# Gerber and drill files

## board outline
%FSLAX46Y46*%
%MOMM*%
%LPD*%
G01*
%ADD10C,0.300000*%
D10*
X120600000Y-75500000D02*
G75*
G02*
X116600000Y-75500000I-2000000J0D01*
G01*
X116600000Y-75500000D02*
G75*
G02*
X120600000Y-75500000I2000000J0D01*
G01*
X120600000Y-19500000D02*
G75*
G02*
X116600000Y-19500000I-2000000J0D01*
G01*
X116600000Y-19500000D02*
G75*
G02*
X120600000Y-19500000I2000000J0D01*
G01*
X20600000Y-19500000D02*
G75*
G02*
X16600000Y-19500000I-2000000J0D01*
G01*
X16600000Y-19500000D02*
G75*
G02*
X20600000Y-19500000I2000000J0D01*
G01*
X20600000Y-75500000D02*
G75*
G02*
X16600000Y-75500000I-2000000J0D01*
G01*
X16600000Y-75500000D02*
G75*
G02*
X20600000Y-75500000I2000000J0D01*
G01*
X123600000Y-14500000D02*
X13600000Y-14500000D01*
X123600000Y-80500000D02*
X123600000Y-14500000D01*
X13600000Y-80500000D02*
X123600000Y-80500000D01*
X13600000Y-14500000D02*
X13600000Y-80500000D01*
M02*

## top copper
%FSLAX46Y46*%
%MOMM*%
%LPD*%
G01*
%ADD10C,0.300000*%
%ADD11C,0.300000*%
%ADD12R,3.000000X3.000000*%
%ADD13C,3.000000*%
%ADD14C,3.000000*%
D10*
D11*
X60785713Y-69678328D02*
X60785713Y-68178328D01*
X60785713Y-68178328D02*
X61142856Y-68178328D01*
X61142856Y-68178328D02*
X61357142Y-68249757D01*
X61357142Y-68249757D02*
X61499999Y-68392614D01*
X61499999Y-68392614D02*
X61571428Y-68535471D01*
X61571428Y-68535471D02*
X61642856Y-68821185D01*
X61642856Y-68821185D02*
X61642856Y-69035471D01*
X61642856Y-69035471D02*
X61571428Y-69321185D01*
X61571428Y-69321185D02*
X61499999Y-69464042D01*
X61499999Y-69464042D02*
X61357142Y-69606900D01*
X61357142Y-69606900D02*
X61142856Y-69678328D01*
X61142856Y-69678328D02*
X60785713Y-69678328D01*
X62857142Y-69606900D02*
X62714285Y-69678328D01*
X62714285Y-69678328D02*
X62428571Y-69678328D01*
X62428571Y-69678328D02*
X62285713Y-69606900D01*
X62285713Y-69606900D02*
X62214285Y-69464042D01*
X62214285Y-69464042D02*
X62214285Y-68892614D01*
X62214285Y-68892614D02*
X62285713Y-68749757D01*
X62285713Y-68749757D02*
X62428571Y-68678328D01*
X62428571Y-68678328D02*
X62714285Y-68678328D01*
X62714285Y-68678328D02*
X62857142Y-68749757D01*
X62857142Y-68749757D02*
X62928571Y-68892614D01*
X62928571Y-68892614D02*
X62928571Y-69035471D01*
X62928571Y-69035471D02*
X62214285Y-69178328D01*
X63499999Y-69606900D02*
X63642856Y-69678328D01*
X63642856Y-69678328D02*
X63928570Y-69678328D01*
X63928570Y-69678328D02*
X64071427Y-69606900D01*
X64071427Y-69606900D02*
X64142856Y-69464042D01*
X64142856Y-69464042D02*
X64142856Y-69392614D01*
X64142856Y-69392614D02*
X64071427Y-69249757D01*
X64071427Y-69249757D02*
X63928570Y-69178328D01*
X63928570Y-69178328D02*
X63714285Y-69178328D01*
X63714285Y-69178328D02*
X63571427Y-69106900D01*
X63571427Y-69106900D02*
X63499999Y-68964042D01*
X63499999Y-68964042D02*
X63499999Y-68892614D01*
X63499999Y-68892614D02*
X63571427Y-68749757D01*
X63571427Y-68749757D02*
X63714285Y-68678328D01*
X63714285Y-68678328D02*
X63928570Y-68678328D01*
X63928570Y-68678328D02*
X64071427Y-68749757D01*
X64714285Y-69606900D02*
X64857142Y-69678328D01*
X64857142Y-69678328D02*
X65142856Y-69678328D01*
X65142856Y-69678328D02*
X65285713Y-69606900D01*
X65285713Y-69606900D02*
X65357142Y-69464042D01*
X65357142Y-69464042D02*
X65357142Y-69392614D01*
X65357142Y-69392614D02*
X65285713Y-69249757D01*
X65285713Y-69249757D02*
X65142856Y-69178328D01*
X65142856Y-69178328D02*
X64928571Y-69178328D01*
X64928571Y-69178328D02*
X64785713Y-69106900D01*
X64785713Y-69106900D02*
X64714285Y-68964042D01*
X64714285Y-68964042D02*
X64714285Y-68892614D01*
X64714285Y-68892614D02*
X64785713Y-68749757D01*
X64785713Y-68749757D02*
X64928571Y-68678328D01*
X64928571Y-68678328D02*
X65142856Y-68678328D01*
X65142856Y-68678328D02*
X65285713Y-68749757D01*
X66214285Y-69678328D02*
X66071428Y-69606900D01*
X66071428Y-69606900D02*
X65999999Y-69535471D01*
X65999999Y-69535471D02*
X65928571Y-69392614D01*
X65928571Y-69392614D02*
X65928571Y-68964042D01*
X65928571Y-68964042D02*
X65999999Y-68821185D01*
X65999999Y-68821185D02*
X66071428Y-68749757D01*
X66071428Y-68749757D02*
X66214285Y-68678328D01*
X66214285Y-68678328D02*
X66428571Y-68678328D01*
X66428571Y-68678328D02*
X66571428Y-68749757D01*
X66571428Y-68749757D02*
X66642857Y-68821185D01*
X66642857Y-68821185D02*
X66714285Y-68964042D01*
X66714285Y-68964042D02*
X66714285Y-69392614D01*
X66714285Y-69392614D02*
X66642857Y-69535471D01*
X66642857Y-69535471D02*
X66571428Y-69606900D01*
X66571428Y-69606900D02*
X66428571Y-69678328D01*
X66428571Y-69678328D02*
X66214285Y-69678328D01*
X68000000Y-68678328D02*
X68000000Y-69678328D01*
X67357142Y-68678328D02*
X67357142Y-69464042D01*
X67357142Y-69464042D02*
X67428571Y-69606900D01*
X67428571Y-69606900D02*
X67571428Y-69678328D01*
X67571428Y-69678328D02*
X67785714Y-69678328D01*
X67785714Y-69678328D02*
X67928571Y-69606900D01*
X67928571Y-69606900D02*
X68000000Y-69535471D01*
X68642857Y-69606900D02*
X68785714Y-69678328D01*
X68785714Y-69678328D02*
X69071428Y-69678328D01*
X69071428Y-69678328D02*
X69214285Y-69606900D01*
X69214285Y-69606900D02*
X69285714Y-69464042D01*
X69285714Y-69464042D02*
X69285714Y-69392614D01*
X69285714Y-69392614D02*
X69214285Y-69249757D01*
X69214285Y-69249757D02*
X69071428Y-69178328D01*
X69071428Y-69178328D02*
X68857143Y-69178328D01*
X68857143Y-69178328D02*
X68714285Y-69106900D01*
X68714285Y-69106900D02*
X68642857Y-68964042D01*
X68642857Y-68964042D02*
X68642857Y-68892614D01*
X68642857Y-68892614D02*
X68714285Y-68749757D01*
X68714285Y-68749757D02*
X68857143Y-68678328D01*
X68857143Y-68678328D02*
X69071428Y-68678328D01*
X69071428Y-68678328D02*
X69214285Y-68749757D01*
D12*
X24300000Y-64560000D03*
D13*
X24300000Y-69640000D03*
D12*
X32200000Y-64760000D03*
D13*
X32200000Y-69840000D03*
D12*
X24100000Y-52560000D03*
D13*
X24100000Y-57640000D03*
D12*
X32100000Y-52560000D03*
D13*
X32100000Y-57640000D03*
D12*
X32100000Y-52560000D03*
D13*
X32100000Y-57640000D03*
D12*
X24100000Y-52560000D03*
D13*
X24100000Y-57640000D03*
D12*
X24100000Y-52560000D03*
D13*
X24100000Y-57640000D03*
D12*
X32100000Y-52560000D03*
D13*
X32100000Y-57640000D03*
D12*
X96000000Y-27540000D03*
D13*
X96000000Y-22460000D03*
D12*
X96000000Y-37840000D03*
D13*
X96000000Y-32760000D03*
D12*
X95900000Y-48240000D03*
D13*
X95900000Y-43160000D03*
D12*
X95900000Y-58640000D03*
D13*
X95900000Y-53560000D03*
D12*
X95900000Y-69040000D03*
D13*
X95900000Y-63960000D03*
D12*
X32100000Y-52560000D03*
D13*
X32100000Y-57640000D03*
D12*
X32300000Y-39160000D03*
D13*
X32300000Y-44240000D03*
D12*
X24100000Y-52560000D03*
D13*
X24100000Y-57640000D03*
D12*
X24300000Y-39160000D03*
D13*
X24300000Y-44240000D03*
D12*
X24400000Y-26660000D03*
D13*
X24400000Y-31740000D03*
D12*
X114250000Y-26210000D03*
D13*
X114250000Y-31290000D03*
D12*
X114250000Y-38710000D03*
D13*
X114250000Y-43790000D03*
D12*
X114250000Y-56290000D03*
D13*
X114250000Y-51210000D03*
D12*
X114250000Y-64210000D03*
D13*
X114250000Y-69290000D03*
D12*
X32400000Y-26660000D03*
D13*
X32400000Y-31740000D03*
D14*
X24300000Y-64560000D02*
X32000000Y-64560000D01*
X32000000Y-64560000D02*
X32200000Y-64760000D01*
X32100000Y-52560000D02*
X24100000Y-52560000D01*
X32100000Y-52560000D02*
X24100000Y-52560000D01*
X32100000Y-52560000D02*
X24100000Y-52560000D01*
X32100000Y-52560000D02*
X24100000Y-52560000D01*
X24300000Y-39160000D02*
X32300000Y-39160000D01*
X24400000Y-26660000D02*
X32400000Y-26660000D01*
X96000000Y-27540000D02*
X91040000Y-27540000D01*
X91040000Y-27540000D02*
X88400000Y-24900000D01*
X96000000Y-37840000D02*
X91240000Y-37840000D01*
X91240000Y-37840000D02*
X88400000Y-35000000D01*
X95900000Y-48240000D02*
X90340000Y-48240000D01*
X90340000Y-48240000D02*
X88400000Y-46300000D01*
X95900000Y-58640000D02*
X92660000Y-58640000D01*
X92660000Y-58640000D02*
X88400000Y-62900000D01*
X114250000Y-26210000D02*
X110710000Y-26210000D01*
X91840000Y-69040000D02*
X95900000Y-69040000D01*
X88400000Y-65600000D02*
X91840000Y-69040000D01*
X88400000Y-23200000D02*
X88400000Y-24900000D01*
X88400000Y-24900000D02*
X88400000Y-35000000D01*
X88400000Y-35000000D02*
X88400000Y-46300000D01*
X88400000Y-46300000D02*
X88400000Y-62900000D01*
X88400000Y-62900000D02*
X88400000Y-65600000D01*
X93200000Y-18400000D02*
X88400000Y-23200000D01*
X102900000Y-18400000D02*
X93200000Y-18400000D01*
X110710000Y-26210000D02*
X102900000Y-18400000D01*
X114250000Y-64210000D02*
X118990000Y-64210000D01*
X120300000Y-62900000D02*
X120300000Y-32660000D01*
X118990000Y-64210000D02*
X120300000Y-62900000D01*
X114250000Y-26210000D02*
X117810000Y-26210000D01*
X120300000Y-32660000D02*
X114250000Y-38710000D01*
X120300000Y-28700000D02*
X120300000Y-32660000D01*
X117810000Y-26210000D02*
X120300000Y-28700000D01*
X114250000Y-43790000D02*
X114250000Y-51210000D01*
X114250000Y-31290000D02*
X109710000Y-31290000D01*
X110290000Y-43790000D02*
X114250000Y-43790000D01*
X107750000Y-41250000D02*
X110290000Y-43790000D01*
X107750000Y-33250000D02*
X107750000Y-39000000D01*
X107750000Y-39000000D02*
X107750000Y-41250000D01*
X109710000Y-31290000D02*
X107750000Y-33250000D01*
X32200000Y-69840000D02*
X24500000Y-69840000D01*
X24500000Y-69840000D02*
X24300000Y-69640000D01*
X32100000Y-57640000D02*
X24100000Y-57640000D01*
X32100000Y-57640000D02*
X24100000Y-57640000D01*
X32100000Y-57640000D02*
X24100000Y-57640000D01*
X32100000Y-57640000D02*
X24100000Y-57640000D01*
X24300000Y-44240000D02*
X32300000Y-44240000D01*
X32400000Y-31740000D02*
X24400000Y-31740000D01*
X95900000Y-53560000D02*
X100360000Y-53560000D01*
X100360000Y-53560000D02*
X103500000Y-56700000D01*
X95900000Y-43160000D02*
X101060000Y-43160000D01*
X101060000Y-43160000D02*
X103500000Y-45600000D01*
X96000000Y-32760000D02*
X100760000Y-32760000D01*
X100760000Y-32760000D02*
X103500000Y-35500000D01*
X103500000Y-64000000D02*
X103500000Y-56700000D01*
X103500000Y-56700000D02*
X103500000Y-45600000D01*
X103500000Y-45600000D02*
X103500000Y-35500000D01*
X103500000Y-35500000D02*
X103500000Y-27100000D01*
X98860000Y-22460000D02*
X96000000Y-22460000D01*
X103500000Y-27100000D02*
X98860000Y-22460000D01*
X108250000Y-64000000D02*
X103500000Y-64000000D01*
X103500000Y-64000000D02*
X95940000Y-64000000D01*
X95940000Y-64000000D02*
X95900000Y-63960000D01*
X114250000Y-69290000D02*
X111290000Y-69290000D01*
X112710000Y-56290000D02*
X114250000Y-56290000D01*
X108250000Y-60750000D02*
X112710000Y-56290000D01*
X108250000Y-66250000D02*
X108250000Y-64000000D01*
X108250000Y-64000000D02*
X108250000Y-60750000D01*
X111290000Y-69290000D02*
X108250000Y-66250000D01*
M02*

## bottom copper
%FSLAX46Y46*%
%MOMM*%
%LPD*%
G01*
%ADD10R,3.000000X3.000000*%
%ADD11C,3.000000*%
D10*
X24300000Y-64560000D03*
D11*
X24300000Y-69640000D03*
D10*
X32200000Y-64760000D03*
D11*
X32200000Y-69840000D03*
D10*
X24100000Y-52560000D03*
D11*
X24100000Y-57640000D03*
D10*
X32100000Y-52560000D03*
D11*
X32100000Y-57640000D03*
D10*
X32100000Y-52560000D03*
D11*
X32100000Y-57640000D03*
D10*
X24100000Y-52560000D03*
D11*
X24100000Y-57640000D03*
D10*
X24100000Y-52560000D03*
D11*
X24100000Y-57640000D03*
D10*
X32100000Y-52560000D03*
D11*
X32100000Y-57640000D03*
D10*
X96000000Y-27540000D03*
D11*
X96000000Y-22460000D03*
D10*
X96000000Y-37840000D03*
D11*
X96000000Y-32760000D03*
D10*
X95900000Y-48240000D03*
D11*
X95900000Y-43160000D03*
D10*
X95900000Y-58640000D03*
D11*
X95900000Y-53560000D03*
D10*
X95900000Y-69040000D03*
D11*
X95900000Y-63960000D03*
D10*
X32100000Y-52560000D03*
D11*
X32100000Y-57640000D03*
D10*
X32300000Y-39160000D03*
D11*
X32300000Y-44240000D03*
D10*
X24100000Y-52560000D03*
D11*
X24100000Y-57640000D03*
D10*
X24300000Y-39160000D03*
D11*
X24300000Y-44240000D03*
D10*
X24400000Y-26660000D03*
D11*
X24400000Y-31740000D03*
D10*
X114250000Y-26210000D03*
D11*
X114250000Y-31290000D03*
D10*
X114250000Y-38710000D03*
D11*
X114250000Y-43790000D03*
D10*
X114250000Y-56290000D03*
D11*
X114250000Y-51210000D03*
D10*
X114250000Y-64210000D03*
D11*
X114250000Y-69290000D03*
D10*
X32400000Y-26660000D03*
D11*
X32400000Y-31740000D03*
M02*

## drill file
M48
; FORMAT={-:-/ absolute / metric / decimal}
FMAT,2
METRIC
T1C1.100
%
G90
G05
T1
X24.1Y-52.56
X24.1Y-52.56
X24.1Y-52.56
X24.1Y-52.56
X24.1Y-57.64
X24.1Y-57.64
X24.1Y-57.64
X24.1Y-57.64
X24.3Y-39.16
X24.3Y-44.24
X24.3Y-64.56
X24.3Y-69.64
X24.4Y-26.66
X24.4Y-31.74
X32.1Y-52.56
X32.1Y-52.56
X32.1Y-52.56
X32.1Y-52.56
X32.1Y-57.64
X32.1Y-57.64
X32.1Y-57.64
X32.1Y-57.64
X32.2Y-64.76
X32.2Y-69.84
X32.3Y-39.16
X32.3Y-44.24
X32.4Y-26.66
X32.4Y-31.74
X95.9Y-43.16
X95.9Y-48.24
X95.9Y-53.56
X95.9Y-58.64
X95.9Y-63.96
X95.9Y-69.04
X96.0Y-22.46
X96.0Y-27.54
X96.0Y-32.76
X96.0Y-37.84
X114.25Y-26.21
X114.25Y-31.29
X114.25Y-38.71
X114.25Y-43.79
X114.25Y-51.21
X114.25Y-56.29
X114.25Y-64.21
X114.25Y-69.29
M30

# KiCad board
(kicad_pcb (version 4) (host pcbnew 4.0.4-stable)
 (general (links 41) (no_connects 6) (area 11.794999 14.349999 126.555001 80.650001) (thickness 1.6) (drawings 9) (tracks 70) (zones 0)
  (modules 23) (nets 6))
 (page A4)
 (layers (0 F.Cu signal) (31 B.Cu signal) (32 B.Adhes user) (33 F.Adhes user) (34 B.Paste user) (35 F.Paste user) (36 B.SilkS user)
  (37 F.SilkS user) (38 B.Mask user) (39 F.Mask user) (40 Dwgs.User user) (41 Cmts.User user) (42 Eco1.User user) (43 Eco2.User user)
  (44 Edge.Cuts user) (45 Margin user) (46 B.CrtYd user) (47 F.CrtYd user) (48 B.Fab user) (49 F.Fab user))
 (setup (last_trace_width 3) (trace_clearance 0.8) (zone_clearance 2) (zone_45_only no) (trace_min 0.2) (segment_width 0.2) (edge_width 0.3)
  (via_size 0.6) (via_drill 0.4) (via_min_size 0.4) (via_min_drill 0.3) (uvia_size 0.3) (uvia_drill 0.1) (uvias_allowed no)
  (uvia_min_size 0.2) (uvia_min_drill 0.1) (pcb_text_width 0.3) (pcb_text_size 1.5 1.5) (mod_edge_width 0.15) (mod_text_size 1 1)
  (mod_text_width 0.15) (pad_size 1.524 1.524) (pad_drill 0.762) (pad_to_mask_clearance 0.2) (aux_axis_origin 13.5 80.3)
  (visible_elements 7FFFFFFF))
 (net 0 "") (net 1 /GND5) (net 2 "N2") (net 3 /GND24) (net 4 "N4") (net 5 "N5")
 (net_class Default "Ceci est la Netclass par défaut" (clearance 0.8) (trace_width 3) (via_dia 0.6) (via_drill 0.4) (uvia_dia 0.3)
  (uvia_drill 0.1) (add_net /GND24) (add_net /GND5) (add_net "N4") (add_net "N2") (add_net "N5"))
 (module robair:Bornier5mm (layer B.Cu) (at 24.3 67.1 270)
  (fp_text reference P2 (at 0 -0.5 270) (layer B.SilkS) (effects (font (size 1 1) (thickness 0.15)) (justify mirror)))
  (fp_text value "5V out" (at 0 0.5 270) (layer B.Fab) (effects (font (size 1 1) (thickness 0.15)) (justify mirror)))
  (pad 1 thru_hole rect (at -2.54 0 270) (size 3 3) (drill 1.1) (layers *.Cu *.Mask) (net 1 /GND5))
  (pad 2 thru_hole circle (at 2.54 0 270) (size 3 3) (drill 1.1) (layers *.Cu *.Mask) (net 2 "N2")))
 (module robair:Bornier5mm (layer F.Cu) (at 32.2 67.3 270)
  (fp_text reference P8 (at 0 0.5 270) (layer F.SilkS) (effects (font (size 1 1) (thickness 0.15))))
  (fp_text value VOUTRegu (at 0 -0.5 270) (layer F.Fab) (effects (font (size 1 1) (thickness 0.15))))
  (pad 1 thru_hole rect (at -2.54 0 270) (size 3 3) (drill 1.1) (layers *.Cu *.Mask) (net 1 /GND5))
  (pad 2 thru_hole circle (at 2.54 0 270) (size 3 3) (drill 1.1) (layers *.Cu *.Mask) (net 2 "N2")))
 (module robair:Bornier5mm (layer B.Cu) (at 24.1 55.1 270)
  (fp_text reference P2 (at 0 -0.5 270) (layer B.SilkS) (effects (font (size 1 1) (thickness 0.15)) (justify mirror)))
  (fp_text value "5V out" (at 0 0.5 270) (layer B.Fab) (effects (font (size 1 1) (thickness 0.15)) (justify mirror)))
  (pad 1 thru_hole rect (at -2.54 0 270) (size 3 3) (drill 1.1) (layers *.Cu *.Mask) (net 1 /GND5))
  (pad 2 thru_hole circle (at 2.54 0 270) (size 3 3) (drill 1.1) (layers *.Cu *.Mask) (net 2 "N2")))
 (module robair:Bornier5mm (layer F.Cu) (at 32.1 55.1 270)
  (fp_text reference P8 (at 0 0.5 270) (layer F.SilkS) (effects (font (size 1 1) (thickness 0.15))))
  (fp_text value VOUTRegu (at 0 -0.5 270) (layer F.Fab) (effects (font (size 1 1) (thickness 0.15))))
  (pad 1 thru_hole rect (at -2.54 0 270) (size 3 3) (drill 1.1) (layers *.Cu *.Mask) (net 1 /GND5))
  (pad 2 thru_hole circle (at 2.54 0 270) (size 3 3) (drill 1.1) (layers *.Cu *.Mask) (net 2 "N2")))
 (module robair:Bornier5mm (layer F.Cu) (at 32.1 55.1 270)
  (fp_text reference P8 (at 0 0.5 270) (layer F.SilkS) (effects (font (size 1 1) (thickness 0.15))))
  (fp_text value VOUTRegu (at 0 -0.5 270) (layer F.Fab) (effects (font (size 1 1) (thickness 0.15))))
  (pad 1 thru_hole rect (at -2.54 0 270) (size 3 3) (drill 1.1) (layers *.Cu *.Mask) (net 1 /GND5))
  (pad 2 thru_hole circle (at 2.54 0 270) (size 3 3) (drill 1.1) (layers *.Cu *.Mask) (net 2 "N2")))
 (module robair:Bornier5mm (layer B.Cu) (at 24.1 55.1 270)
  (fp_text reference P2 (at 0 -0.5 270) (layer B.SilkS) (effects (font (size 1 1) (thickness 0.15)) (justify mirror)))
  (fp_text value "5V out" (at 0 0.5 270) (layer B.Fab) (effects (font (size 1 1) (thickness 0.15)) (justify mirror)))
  (pad 1 thru_hole rect (at -2.54 0 270) (size 3 3) (drill 1.1) (layers *.Cu *.Mask) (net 1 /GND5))
  (pad 2 thru_hole circle (at 2.54 0 270) (size 3 3) (drill 1.1) (layers *.Cu *.Mask) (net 2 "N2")))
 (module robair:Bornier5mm (layer B.Cu) (at 24.1 55.1 270)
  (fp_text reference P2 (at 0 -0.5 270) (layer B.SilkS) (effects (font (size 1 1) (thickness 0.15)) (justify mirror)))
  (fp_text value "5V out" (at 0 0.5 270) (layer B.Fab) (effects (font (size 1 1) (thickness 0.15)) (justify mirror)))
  (pad 1 thru_hole rect (at -2.54 0 270) (size 3 3) (drill 1.1) (layers *.Cu *.Mask) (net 1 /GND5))
  (pad 2 thru_hole circle (at 2.54 0 270) (size 3 3) (drill 1.1) (layers *.Cu *.Mask) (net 2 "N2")))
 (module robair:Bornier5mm (layer F.Cu) (at 32.1 55.1 270)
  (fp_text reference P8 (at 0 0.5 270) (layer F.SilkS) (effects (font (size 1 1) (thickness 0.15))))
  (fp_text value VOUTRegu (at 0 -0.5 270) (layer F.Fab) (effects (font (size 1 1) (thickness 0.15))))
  (pad 1 thru_hole rect (at -2.54 0 270) (size 3 3) (drill 1.1) (layers *.Cu *.Mask) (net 1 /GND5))
  (pad 2 thru_hole circle (at 2.54 0 270) (size 3 3) (drill 1.1) (layers *.Cu *.Mask) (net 2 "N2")))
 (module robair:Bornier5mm (layer F.Cu) (at 96 25 90)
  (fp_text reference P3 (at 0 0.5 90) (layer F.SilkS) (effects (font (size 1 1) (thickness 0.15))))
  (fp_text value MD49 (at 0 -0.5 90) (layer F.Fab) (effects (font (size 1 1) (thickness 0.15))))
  (pad 1 thru_hole rect (at -2.54 0 90) (size 3 3) (drill 1.1) (layers *.Cu *.Mask) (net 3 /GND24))
  (pad 2 thru_hole circle (at 2.54 0 90) (size 3 3) (drill 1.1) (layers *.Cu *.Mask) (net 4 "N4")))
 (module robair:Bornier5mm (layer F.Cu) (at 96 35.3 90)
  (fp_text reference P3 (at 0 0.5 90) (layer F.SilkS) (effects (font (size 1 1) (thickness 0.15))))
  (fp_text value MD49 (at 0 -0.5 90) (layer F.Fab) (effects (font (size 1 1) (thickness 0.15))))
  (pad 1 thru_hole rect (at -2.54 0 90) (size 3 3) (drill 1.1) (layers *.Cu *.Mask) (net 3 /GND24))
  (pad 2 thru_hole circle (at 2.54 0 90) (size 3 3) (drill 1.1) (layers *.Cu *.Mask) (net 4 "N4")))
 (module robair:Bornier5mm (layer F.Cu) (at 95.9 45.7 90)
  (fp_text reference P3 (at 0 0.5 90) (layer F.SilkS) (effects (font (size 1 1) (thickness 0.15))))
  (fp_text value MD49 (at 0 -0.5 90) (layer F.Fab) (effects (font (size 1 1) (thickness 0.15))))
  (pad 1 thru_hole rect (at -2.54 0 90) (size 3 3) (drill 1.1) (layers *.Cu *.Mask) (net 3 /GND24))
  (pad 2 thru_hole circle (at 2.54 0 90) (size 3 3) (drill 1.1) (layers *.Cu *.Mask) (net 4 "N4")))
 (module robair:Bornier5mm (layer F.Cu) (at 95.9 56.1 90)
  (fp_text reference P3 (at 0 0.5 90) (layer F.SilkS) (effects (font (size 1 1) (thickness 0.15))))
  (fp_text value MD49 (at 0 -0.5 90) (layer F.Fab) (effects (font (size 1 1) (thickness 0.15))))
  (pad 1 thru_hole rect (at -2.54 0 90) (size 3 3) (drill 1.1) (layers *.Cu *.Mask) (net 3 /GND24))
  (pad 2 thru_hole circle (at 2.54 0 90) (size 3 3) (drill 1.1) (layers *.Cu *.Mask) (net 4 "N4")))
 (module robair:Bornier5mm (layer F.Cu) (at 95.9 66.5 90)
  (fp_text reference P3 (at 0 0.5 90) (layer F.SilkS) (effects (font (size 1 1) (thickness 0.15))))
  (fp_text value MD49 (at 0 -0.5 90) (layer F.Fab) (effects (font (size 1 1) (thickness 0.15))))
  (pad 1 thru_hole rect (at -2.54 0 90) (size 3 3) (drill 1.1) (layers *.Cu *.Mask) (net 3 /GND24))
  (pad 2 thru_hole circle (at 2.54 0 90) (size 3 3) (drill 1.1) (layers *.Cu *.Mask) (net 4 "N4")))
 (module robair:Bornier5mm (layer F.Cu) (at 32.1 55.1 270)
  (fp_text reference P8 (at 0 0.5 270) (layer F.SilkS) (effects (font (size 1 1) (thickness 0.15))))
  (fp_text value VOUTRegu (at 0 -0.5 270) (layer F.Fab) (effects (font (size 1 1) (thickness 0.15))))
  (pad 1 thru_hole rect (at -2.54 0 270) (size 3 3) (drill 1.1) (layers *.Cu *.Mask) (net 1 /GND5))
  (pad 2 thru_hole circle (at 2.54 0 270) (size 3 3) (drill 1.1) (layers *.Cu *.Mask) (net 2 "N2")))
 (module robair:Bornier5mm (layer F.Cu) (at 32.3 41.7 270)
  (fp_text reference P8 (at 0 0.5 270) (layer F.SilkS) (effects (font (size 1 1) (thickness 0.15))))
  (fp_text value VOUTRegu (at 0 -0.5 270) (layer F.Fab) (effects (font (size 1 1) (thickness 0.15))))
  (pad 1 thru_hole rect (at -2.54 0 270) (size 3 3) (drill 1.1) (layers *.Cu *.Mask) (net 1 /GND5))
  (pad 2 thru_hole circle (at 2.54 0 270) (size 3 3) (drill 1.1) (layers *.Cu *.Mask) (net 2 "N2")))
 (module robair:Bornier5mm (layer B.Cu) (at 24.1 55.1 270)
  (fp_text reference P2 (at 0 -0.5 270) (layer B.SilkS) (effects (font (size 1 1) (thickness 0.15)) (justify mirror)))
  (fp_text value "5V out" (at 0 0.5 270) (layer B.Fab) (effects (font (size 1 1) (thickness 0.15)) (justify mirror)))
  (pad 1 thru_hole rect (at -2.54 0 270) (size 3 3) (drill 1.1) (layers *.Cu *.Mask) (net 1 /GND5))
  (pad 2 thru_hole circle (at 2.54 0 270) (size 3 3) (drill 1.1) (layers *.Cu *.Mask) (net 2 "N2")))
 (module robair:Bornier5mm (layer B.Cu) (at 24.3 41.7 270)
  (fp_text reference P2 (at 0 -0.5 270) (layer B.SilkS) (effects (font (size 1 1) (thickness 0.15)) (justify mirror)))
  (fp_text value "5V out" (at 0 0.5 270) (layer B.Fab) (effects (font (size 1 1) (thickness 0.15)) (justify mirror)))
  (pad 1 thru_hole rect (at -2.54 0 270) (size 3 3) (drill 1.1) (layers *.Cu *.Mask) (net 1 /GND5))
  (pad 2 thru_hole circle (at 2.54 0 270) (size 3 3) (drill 1.1) (layers *.Cu *.Mask) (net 2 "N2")))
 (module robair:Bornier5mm (layer B.Cu) (at 24.4 29.2 270)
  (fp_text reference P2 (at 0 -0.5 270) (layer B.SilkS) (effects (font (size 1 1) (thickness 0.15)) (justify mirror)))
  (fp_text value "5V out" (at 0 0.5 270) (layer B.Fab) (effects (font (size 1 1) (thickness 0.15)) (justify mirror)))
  (pad 1 thru_hole rect (at -2.54 0 270) (size 3 3) (drill 1.1) (layers *.Cu *.Mask) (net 1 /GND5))
  (pad 2 thru_hole circle (at 2.54 0 270) (size 3 3) (drill 1.1) (layers *.Cu *.Mask) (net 2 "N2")))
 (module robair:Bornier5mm (layer F.Cu) (at 114.25 28.75 270)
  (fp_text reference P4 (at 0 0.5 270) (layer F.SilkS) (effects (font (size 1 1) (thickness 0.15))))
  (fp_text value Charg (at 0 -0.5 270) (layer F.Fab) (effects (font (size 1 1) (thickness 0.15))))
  (pad 1 thru_hole rect (at -2.54 0 270) (size 3 3) (drill 1.1) (layers *.Cu *.Mask) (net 3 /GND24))
  (pad 2 thru_hole circle (at 2.54 0 270) (size 3 3) (drill 1.1) (layers *.Cu *.Mask) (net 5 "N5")))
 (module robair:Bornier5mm (layer F.Cu) (at 114.25 41.25 270)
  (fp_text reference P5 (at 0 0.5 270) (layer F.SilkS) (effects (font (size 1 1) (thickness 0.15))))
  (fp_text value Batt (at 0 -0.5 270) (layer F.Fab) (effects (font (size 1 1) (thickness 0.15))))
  (pad 1 thru_hole rect (at -2.54 0 270) (size 3 3) (drill 1.1) (layers *.Cu *.Mask) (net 3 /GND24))
  (pad 2 thru_hole circle (at 2.54 0 270) (size 3 3) (drill 1.1) (layers *.Cu *.Mask) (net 5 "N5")))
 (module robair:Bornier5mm (layer B.Cu) (at 114.25 53.75 90)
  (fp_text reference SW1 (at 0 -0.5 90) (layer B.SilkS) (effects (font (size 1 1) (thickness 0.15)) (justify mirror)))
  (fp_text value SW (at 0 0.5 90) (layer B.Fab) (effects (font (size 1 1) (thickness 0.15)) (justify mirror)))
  (pad 1 thru_hole rect (at -2.54 0 90) (size 3 3) (drill 1.1) (layers *.Cu *.Mask) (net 4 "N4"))
  (pad 2 thru_hole circle (at 2.54 0 90) (size 3 3) (drill 1.1) (layers *.Cu *.Mask) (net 5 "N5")))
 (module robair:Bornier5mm (layer F.Cu) (at 114.25 66.75 270)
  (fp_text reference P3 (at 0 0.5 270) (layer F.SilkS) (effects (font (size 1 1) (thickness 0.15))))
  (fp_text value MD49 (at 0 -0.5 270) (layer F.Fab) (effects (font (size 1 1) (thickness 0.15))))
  (pad 1 thru_hole rect (at -2.54 0 270) (size 3 3) (drill 1.1) (layers *.Cu *.Mask) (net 3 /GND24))
  (pad 2 thru_hole circle (at 2.54 0 270) (size 3 3) (drill 1.1) (layers *.Cu *.Mask) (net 4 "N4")))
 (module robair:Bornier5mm (layer F.Cu) (at 32.4 29.2 270)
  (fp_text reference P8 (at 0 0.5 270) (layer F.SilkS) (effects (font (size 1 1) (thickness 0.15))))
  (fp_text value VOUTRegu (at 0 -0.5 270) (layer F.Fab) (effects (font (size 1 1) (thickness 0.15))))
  (pad 1 thru_hole rect (at -2.54 0 270) (size 3 3) (drill 1.1) (layers *.Cu *.Mask) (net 1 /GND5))
  (pad 2 thru_hole circle (at 2.54 0 270) (size 3 3) (drill 1.1) (layers *.Cu *.Mask) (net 2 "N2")))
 (gr_circle (center 118.6 75.5) (end 118.6 77.5) (layer Edge.Cuts) (width 0.3))
 (gr_circle (center 118.6 19.5) (end 120.6 19.5) (layer Edge.Cuts) (width 0.3))
 (gr_circle (center 18.6 19.5) (end 16.6 19.5) (layer Edge.Cuts) (width 0.3))
 (gr_circle (center 18.6 75.5) (end 16.6 75.5) (layer Edge.Cuts) (width 0.3))
 (gr_line (start 123.6 14.5) (end 13.6 14.5) (angle 90) (layer Edge.Cuts) (width 0.3))
 (gr_line (start 123.6 80.5) (end 123.6 14.5) (angle 90) (layer Edge.Cuts) (width 0.3))
 (gr_line (start 13.6 80.5) (end 123.6 80.5) (angle 90) (layer Edge.Cuts) (width 0.3))
 (gr_line (start 13.6 14.5) (end 13.6 80.5) (angle 90) (layer Edge.Cuts) (width 0.3))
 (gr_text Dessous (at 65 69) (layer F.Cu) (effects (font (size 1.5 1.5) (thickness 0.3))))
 (segment (start 24.3 64.56) (end 32 64.56) (width 3) (layer F.Cu) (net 1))
 (segment (start 32 64.56) (end 32.2 64.76) (width 3) (layer F.Cu) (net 1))
 (segment (start 32.1 52.56) (end 24.1 52.56) (width 3) (layer F.Cu) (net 1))
 (segment (start 32.1 52.56) (end 24.1 52.56) (width 3) (layer F.Cu) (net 1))
 (segment (start 32.1 52.56) (end 24.1 52.56) (width 3) (layer F.Cu) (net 1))
 (segment (start 32.1 52.56) (end 24.1 52.56) (width 3) (layer F.Cu) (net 1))
 (segment (start 24.3 39.16) (end 32.3 39.16) (width 3) (layer F.Cu) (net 1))
 (segment (start 24.4 26.66) (end 32.4 26.66) (width 3) (layer F.Cu) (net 1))
 (segment (start 96 27.54) (end 91.04 27.54) (width 3) (layer F.Cu) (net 3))
 (segment (start 91.04 27.54) (end 88.4 24.9) (width 3) (layer F.Cu) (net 3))
 (segment (start 96 37.84) (end 91.24 37.84) (width 3) (layer F.Cu) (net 3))
 (segment (start 91.24 37.84) (end 88.4 35) (width 3) (layer F.Cu) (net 3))
 (segment (start 95.9 48.24) (end 90.34 48.24) (width 3) (layer F.Cu) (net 3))
 (segment (start 90.34 48.24) (end 88.4 46.3) (width 3) (layer F.Cu) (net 3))
 (segment (start 95.9 58.64) (end 92.66 58.64) (width 3) (layer F.Cu) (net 3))
 (segment (start 92.66 58.64) (end 88.4 62.9) (width 3) (layer F.Cu) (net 3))
 (segment (start 114.25 26.21) (end 110.71 26.21) (width 3) (layer F.Cu) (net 3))
 (segment (start 91.84 69.04) (end 95.9 69.04) (width 3) (layer F.Cu) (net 3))
 (segment (start 88.4 65.6) (end 91.84 69.04) (width 3) (layer F.Cu) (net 3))
 (segment (start 88.4 23.2) (end 88.4 24.9) (width 3) (layer F.Cu) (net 3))
 (segment (start 88.4 24.9) (end 88.4 35) (width 3) (layer F.Cu) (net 3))
 (segment (start 88.4 35) (end 88.4 46.3) (width 3) (layer F.Cu) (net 3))
 (segment (start 88.4 46.3) (end 88.4 62.9) (width 3) (layer F.Cu) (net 3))
 (segment (start 88.4 62.9) (end 88.4 65.6) (width 3) (layer F.Cu) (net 3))
 (segment (start 93.2 18.4) (end 88.4 23.2) (width 3) (layer F.Cu) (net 3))
 (segment (start 102.9 18.4) (end 93.2 18.4) (width 3) (layer F.Cu) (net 3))
 (segment (start 110.71 26.21) (end 102.9 18.4) (width 3) (layer F.Cu) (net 3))
 (segment (start 114.25 64.21) (end 118.99 64.21) (width 3) (layer F.Cu) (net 3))
 (segment (start 120.3 62.9) (end 120.3 32.66) (width 3) (layer F.Cu) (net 3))
 (segment (start 118.99 64.21) (end 120.3 62.9) (width 3) (layer F.Cu) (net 3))
 (segment (start 114.25 26.21) (end 117.81 26.21) (width 3) (layer F.Cu) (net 3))
 (segment (start 120.3 32.66) (end 114.25 38.71) (width 3) (layer F.Cu) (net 3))
 (segment (start 120.3 28.7) (end 120.3 32.66) (width 3) (layer F.Cu) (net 3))
 (segment (start 117.81 26.21) (end 120.3 28.7) (width 3) (layer F.Cu) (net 3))
 (segment (start 114.25 43.79) (end 114.25 51.21) (width 3) (layer F.Cu) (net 5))
 (segment (start 114.25 31.29) (end 109.71 31.29) (width 3) (layer F.Cu) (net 5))
 (segment (start 110.29 43.79) (end 114.25 43.79) (width 3) (layer F.Cu) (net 5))
 (segment (start 107.75 41.25) (end 110.29 43.79) (width 3) (layer F.Cu) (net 5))
 (segment (start 107.75 33.25) (end 107.75 39) (width 3) (layer F.Cu) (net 5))
 (segment (start 107.75 39) (end 107.75 41.25) (width 3) (layer F.Cu) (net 5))
 (segment (start 109.71 31.29) (end 107.75 33.25) (width 3) (layer F.Cu) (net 5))
 (segment (start 32.2 69.84) (end 24.5 69.84) (width 3) (layer F.Cu) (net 2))
 (segment (start 24.5 69.84) (end 24.3 69.64) (width 3) (layer F.Cu) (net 2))
 (segment (start 32.1 57.64) (end 24.1 57.64) (width 3) (layer F.Cu) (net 2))
 (segment (start 32.1 57.64) (end 24.1 57.64) (width 3) (layer F.Cu) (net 2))
 (segment (start 32.1 57.64) (end 24.1 57.64) (width 3) (layer F.Cu) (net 2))
 (segment (start 32.1 57.64) (end 24.1 57.64) (width 3) (layer F.Cu) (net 2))
 (segment (start 24.3 44.24) (end 32.3 44.24) (width 3) (layer F.Cu) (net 2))
 (segment (start 32.4 31.74) (end 24.4 31.74) (width 3) (layer F.Cu) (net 2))
 (segment (start 95.9 53.56) (end 100.36 53.56) (width 3) (layer F.Cu) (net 4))
 (segment (start 100.36 53.56) (end 103.5 56.7) (width 3) (layer F.Cu) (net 4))
 (segment (start 95.9 43.16) (end 101.06 43.16) (width 3) (layer F.Cu) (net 4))
 (segment (start 101.06 43.16) (end 103.5 45.6) (width 3) (layer F.Cu) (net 4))
 (segment (start 96 32.76) (end 100.76 32.76) (width 3) (layer F.Cu) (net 4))
 (segment (start 100.76 32.76) (end 103.5 35.5) (width 3) (layer F.Cu) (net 4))
 (segment (start 103.5 64) (end 103.5 56.7) (width 3) (layer F.Cu) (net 4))
 (segment (start 103.5 56.7) (end 103.5 45.6) (width 3) (layer F.Cu) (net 4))
 (segment (start 103.5 45.6) (end 103.5 35.5) (width 3) (layer F.Cu) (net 4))
 (segment (start 103.5 35.5) (end 103.5 27.1) (width 3) (layer F.Cu) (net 4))
 (segment (start 98.86 22.46) (end 96 22.46) (width 3) (layer F.Cu) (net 4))
 (segment (start 103.5 27.1) (end 98.86 22.46) (width 3) (layer F.Cu) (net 4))
 (segment (start 108.25 64) (end 103.5 64) (width 3) (layer F.Cu) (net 4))
 (segment (start 103.5 64) (end 95.94 64) (width 3) (layer F.Cu) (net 4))
 (segment (start 95.94 64) (end 95.9 63.96) (width 3) (layer F.Cu) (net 4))
 (segment (start 114.25 69.29) (end 111.29 69.29) (width 3) (layer F.Cu) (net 4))
 (segment (start 112.71 56.29) (end 114.25 56.29) (width 3) (layer F.Cu) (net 4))
 (segment (start 108.25 60.75) (end 112.71 56.29) (width 3) (layer F.Cu) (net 4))
 (segment (start 108.25 66.25) (end 108.25 64) (width 3) (layer F.Cu) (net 4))
 (segment (start 108.25 64) (end 108.25 60.75) (width 3) (layer F.Cu) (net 4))
 (segment (start 111.29 69.29) (end 108.25 66.25) (width 3) (layer F.Cu) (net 4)))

